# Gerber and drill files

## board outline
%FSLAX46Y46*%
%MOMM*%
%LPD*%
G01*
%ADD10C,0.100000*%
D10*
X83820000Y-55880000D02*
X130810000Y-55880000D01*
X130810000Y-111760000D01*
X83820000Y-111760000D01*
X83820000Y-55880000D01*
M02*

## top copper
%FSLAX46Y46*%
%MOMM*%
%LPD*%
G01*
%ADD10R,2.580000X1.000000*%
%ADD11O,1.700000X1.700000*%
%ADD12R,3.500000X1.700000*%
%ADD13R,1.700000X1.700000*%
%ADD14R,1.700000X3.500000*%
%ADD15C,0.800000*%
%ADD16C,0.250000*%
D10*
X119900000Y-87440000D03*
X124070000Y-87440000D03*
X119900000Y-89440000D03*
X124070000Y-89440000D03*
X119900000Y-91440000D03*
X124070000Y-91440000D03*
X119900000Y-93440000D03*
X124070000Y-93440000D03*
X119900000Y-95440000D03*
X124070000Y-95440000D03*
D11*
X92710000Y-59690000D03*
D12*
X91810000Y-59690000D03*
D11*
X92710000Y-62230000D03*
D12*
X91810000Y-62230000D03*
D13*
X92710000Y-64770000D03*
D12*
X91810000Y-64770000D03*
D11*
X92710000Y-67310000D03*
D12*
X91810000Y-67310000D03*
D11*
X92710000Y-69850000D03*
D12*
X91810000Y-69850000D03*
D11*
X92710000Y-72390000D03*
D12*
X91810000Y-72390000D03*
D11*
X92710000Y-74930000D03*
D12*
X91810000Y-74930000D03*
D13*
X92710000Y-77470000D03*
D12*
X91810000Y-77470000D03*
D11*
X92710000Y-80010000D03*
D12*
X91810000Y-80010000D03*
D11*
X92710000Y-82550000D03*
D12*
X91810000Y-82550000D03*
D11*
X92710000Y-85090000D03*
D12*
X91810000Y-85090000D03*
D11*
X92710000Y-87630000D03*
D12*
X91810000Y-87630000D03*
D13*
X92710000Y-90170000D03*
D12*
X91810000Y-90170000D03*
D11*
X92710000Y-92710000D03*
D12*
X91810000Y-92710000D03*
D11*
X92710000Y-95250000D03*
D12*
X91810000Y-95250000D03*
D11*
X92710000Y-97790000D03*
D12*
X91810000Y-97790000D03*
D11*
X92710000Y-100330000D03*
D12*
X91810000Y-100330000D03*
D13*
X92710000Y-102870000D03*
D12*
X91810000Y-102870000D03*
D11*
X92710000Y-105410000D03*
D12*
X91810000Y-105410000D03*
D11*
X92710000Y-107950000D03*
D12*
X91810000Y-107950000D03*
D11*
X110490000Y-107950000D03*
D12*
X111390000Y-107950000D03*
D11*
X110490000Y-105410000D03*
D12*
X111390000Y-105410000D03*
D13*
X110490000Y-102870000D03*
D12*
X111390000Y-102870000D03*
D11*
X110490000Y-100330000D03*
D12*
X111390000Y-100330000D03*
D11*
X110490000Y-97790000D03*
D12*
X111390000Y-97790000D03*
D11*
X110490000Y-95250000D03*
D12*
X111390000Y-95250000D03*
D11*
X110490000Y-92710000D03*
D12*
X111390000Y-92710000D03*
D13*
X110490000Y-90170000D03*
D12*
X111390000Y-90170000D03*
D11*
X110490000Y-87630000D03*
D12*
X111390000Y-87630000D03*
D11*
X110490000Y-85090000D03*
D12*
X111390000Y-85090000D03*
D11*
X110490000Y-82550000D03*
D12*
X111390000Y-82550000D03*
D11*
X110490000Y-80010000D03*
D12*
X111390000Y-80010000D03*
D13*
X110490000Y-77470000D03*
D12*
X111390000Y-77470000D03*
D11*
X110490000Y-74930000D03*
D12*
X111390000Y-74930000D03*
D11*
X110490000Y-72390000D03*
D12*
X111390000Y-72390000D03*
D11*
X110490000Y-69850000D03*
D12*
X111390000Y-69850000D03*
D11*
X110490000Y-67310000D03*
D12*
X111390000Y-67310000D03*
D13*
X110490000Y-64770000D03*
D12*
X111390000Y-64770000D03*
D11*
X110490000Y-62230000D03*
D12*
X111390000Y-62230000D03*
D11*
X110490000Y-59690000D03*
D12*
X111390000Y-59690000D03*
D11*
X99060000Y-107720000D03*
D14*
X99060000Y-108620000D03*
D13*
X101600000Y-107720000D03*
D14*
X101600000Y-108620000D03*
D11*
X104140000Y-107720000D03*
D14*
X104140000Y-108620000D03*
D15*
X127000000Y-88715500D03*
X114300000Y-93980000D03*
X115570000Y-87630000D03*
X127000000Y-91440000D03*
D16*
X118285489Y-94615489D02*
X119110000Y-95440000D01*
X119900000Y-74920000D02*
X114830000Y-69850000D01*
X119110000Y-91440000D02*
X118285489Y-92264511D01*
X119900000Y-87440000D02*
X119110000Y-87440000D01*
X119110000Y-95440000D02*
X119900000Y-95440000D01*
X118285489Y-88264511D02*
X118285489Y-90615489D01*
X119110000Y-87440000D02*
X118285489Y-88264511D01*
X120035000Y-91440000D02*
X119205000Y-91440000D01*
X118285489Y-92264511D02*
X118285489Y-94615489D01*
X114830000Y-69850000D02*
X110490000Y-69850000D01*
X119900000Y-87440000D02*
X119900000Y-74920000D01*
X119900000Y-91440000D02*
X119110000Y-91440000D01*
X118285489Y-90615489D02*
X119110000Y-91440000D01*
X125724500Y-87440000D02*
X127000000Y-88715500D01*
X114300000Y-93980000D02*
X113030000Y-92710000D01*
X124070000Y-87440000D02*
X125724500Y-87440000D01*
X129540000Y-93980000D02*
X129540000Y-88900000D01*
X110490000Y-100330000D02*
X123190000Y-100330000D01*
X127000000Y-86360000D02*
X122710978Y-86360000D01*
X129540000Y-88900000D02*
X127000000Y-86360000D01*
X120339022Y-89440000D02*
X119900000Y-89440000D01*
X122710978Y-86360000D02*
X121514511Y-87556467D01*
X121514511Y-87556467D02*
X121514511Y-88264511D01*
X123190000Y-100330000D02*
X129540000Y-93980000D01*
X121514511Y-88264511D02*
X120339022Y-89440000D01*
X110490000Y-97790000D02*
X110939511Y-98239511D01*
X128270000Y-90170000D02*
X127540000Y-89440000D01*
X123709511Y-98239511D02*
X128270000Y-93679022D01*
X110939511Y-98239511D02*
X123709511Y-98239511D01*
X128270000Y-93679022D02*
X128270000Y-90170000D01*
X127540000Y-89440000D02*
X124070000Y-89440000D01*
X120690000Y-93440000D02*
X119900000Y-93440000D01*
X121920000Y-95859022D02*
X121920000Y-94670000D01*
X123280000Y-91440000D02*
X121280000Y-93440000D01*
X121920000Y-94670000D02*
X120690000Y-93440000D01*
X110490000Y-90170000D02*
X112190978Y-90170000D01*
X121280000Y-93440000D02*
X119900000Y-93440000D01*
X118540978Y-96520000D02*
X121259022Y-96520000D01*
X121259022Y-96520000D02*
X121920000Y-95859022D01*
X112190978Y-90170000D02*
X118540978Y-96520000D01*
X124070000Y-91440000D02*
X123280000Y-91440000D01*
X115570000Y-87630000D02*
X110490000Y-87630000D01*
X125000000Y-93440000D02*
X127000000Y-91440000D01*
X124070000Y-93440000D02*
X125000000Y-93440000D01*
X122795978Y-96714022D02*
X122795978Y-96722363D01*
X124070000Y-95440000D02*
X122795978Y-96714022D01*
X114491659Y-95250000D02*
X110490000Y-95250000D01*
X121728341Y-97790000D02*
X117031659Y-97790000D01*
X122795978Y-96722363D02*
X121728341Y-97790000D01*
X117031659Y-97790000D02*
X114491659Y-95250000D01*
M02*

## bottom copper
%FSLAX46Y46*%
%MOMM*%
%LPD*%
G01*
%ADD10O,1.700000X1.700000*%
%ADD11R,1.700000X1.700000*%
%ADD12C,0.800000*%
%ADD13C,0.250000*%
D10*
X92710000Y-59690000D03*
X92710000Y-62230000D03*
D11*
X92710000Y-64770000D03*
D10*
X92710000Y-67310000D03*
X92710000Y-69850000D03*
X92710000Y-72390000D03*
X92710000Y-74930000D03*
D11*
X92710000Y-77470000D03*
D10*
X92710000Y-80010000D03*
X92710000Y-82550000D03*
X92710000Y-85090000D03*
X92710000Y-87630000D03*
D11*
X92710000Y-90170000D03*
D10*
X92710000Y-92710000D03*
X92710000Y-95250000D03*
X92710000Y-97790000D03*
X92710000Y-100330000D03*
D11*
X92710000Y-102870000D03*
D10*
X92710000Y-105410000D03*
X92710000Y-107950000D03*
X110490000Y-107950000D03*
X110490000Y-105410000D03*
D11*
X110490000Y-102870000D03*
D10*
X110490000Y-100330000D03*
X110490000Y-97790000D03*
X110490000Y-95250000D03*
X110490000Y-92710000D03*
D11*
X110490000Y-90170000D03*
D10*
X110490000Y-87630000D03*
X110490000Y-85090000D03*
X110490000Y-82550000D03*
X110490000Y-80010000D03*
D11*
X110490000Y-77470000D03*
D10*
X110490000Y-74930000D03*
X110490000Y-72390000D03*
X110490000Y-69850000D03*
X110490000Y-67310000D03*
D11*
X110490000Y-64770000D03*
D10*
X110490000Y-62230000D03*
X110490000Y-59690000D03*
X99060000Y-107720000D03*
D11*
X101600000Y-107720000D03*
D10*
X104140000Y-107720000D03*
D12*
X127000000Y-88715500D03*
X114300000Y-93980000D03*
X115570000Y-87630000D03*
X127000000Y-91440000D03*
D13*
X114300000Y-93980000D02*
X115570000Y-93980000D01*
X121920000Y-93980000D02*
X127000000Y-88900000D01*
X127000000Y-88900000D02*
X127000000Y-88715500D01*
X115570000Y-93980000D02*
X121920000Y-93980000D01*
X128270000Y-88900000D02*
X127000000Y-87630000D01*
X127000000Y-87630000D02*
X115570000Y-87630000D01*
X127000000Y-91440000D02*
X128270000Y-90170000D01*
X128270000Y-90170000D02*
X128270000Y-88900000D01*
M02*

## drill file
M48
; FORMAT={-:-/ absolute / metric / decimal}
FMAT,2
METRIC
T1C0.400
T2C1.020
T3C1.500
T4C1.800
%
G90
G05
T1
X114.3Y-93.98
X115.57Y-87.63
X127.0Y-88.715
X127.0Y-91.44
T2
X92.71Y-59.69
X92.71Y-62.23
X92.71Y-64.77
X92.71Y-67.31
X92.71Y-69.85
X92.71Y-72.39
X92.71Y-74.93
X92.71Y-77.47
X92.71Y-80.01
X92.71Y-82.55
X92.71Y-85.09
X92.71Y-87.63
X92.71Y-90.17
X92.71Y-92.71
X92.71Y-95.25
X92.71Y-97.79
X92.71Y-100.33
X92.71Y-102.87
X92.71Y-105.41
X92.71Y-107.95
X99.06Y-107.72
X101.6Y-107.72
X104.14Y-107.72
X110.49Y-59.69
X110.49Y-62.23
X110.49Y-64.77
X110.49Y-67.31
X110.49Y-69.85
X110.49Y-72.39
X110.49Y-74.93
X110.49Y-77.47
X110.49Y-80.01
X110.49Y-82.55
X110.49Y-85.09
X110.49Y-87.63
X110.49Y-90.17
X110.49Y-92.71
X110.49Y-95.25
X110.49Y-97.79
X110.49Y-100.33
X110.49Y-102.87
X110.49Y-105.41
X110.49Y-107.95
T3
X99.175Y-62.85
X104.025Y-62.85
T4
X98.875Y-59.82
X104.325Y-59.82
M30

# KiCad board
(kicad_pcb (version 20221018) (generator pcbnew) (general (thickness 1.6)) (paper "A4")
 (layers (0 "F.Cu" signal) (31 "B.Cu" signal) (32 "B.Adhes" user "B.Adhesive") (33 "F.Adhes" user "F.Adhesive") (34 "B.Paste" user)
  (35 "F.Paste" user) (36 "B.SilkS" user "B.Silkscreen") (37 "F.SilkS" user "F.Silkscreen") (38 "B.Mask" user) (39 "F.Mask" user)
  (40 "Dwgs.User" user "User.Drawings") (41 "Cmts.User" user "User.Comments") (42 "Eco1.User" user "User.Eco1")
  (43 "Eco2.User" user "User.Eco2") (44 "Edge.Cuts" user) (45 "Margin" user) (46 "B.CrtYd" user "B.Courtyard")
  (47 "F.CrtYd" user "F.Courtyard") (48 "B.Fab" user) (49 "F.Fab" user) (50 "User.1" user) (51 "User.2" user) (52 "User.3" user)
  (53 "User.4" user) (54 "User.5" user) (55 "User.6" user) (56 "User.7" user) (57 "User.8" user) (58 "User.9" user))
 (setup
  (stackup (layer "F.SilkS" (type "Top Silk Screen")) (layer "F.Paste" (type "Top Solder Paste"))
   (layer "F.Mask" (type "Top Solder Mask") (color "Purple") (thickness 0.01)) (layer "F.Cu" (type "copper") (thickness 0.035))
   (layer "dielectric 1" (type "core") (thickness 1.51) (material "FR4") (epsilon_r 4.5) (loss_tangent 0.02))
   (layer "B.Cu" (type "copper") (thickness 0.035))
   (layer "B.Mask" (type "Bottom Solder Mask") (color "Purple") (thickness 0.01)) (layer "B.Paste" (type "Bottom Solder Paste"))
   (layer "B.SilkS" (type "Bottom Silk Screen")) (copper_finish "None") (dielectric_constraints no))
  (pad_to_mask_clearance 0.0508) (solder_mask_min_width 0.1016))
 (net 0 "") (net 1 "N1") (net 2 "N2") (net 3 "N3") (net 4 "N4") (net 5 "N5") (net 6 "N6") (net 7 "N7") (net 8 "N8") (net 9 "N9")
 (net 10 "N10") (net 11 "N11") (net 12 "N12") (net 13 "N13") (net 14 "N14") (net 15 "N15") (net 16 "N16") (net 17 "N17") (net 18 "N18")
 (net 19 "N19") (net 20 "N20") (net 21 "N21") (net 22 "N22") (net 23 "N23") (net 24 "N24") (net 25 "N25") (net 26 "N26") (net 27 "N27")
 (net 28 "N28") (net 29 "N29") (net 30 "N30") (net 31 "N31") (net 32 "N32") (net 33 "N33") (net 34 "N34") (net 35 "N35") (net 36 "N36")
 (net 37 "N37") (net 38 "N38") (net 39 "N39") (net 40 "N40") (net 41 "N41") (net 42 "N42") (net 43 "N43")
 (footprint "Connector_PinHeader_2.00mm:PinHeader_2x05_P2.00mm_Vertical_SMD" (layer "F.Cu") (at 121.985 91.44)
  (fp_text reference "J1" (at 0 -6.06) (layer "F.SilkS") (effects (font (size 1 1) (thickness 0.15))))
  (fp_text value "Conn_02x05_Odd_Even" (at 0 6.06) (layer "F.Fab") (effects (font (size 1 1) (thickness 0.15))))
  (pad "1" smd rect (at -2.085 -4) (size 2.58 1) (layers "F.Cu" "F.Paste" "F.Mask") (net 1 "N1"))
  (pad "2" smd rect (at 2.085 -4) (size 2.58 1) (layers "F.Cu" "F.Paste" "F.Mask") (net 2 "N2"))
  (pad "3" smd rect (at -2.085 -2) (size 2.58 1) (layers "F.Cu" "F.Paste" "F.Mask") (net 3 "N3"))
  (pad "4" smd rect (at 2.085 -2) (size 2.58 1) (layers "F.Cu" "F.Paste" "F.Mask") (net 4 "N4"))
  (pad "5" smd rect (at -2.085 0) (size 2.58 1) (layers "F.Cu" "F.Paste" "F.Mask") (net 1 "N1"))
  (pad "6" smd rect (at 2.085 0) (size 2.58 1) (layers "F.Cu" "F.Paste" "F.Mask") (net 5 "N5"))
  (pad "7" smd rect (at -2.085 2) (size 2.58 1) (layers "F.Cu" "F.Paste" "F.Mask") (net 5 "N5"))
  (pad "8" smd rect (at 2.085 2) (size 2.58 1) (layers "F.Cu" "F.Paste" "F.Mask") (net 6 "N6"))
  (pad "9" smd rect (at -2.085 4) (size 2.58 1) (layers "F.Cu" "F.Paste" "F.Mask") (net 1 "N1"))
  (pad "10" smd rect (at 2.085 4) (size 2.58 1) (layers "F.Cu" "F.Paste" "F.Mask") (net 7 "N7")))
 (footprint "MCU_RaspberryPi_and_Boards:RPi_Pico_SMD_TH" (layer "F.Cu") (at 101.6 83.82)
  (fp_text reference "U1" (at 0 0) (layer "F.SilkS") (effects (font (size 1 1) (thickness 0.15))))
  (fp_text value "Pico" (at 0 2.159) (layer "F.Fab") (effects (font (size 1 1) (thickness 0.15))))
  (pad "" np_thru_hole oval (at -2.725 -24) (size 1.8 1.8) (drill 1.8) (layers "*.Cu" "*.Mask"))
  (pad "" np_thru_hole oval (at -2.425 -20.97) (size 1.5 1.5) (drill 1.5) (layers "*.Cu" "*.Mask"))
  (pad "" np_thru_hole oval (at 2.425 -20.97) (size 1.5 1.5) (drill 1.5) (layers "*.Cu" "*.Mask"))
  (pad "" np_thru_hole oval (at 2.725 -24) (size 1.8 1.8) (drill 1.8) (layers "*.Cu" "*.Mask"))
  (pad "1" thru_hole oval (at -8.89 -24.13) (size 1.7 1.7) (drill 1.02) (layers "*.Cu" "*.Mask") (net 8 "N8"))
  (pad "1" smd rect (at -8.89 -24.13) (size 3.5 1.7) (drill (offset -0.9 0)) (layers "F.Cu" "F.Mask") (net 8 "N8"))
  (pad "2" thru_hole oval (at -8.89 -21.59) (size 1.7 1.7) (drill 1.02) (layers "*.Cu" "*.Mask") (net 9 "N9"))
  (pad "2" smd rect (at -8.89 -21.59) (size 3.5 1.7) (drill (offset -0.9 0)) (layers "F.Cu" "F.Mask") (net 9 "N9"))
  (pad "3" thru_hole rect (at -8.89 -19.05) (size 1.7 1.7) (drill 1.02) (layers "*.Cu" "*.Mask") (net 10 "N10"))
  (pad "3" smd rect (at -8.89 -19.05) (size 3.5 1.7) (drill (offset -0.9 0)) (layers "F.Cu" "F.Mask") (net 10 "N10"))
  (pad "4" thru_hole oval (at -8.89 -16.51) (size 1.7 1.7) (drill 1.02) (layers "*.Cu" "*.Mask") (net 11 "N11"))
  (pad "4" smd rect (at -8.89 -16.51) (size 3.5 1.7) (drill (offset -0.9 0)) (layers "F.Cu" "F.Mask") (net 11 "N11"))
  (pad "5" thru_hole oval (at -8.89 -13.97) (size 1.7 1.7) (drill 1.02) (layers "*.Cu" "*.Mask") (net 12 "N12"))
  (pad "5" smd rect (at -8.89 -13.97) (size 3.5 1.7) (drill (offset -0.9 0)) (layers "F.Cu" "F.Mask") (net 12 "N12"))
  (pad "6" thru_hole oval (at -8.89 -11.43) (size 1.7 1.7) (drill 1.02) (layers "*.Cu" "*.Mask") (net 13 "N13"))
  (pad "6" smd rect (at -8.89 -11.43) (size 3.5 1.7) (drill (offset -0.9 0)) (layers "F.Cu" "F.Mask") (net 13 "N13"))
  (pad "7" thru_hole oval (at -8.89 -8.89) (size 1.7 1.7) (drill 1.02) (layers "*.Cu" "*.Mask") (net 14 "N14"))
  (pad "7" smd rect (at -8.89 -8.89) (size 3.5 1.7) (drill (offset -0.9 0)) (layers "F.Cu" "F.Mask") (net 14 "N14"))
  (pad "8" thru_hole rect (at -8.89 -6.35) (size 1.7 1.7) (drill 1.02) (layers "*.Cu" "*.Mask") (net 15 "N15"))
  (pad "8" smd rect (at -8.89 -6.35) (size 3.5 1.7) (drill (offset -0.9 0)) (layers "F.Cu" "F.Mask") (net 15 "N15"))
  (pad "9" thru_hole oval (at -8.89 -3.81) (size 1.7 1.7) (drill 1.02) (layers "*.Cu" "*.Mask") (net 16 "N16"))
  (pad "9" smd rect (at -8.89 -3.81) (size 3.5 1.7) (drill (offset -0.9 0)) (layers "F.Cu" "F.Mask") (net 16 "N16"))
  (pad "10" thru_hole oval (at -8.89 -1.27) (size 1.7 1.7) (drill 1.02) (layers "*.Cu" "*.Mask") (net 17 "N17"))
  (pad "10" smd rect (at -8.89 -1.27) (size 3.5 1.7) (drill (offset -0.9 0)) (layers "F.Cu" "F.Mask") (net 17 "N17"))
  (pad "11" thru_hole oval (at -8.89 1.27) (size 1.7 1.7) (drill 1.02) (layers "*.Cu" "*.Mask") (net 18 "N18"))
  (pad "11" smd rect (at -8.89 1.27) (size 3.5 1.7) (drill (offset -0.9 0)) (layers "F.Cu" "F.Mask") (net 18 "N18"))
  (pad "12" thru_hole oval (at -8.89 3.81) (size 1.7 1.7) (drill 1.02) (layers "*.Cu" "*.Mask") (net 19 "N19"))
  (pad "12" smd rect (at -8.89 3.81) (size 3.5 1.7) (drill (offset -0.9 0)) (layers "F.Cu" "F.Mask") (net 19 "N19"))
  (pad "13" thru_hole rect (at -8.89 6.35) (size 1.7 1.7) (drill 1.02) (layers "*.Cu" "*.Mask") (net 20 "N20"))
  (pad "13" smd rect (at -8.89 6.35) (size 3.5 1.7) (drill (offset -0.9 0)) (layers "F.Cu" "F.Mask") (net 20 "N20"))
  (pad "14" thru_hole oval (at -8.89 8.89) (size 1.7 1.7) (drill 1.02) (layers "*.Cu" "*.Mask") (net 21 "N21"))
  (pad "14" smd rect (at -8.89 8.89) (size 3.5 1.7) (drill (offset -0.9 0)) (layers "F.Cu" "F.Mask") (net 21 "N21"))
  (pad "15" thru_hole oval (at -8.89 11.43) (size 1.7 1.7) (drill 1.02) (layers "*.Cu" "*.Mask") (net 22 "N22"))
  (pad "15" smd rect (at -8.89 11.43) (size 3.5 1.7) (drill (offset -0.9 0)) (layers "F.Cu" "F.Mask") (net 22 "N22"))
  (pad "16" thru_hole oval (at -8.89 13.97) (size 1.7 1.7) (drill 1.02) (layers "*.Cu" "*.Mask") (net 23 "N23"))
  (pad "16" smd rect (at -8.89 13.97) (size 3.5 1.7) (drill (offset -0.9 0)) (layers "F.Cu" "F.Mask") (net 23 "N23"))
  (pad "17" thru_hole oval (at -8.89 16.51) (size 1.7 1.7) (drill 1.02) (layers "*.Cu" "*.Mask") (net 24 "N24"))
  (pad "17" smd rect (at -8.89 16.51) (size 3.5 1.7) (drill (offset -0.9 0)) (layers "F.Cu" "F.Mask") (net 24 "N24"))
  (pad "18" thru_hole rect (at -8.89 19.05) (size 1.7 1.7) (drill 1.02) (layers "*.Cu" "*.Mask") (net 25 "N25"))
  (pad "18" smd rect (at -8.89 19.05) (size 3.5 1.7) (drill (offset -0.9 0)) (layers "F.Cu" "F.Mask") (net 25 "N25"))
  (pad "19" thru_hole oval (at -8.89 21.59) (size 1.7 1.7) (drill 1.02) (layers "*.Cu" "*.Mask") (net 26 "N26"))
  (pad "19" smd rect (at -8.89 21.59) (size 3.5 1.7) (drill (offset -0.9 0)) (layers "F.Cu" "F.Mask") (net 26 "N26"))
  (pad "20" thru_hole oval (at -8.89 24.13) (size 1.7 1.7) (drill 1.02) (layers "*.Cu" "*.Mask") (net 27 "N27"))
  (pad "20" smd rect (at -8.89 24.13) (size 3.5 1.7) (drill (offset -0.9 0)) (layers "F.Cu" "F.Mask") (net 27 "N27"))
  (pad "21" thru_hole oval (at 8.89 24.13) (size 1.7 1.7) (drill 1.02) (layers "*.Cu" "*.Mask") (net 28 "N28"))
  (pad "21" smd rect (at 8.89 24.13) (size 3.5 1.7) (drill (offset 0.9 0)) (layers "F.Cu" "F.Mask") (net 28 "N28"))
  (pad "22" thru_hole oval (at 8.89 21.59) (size 1.7 1.7) (drill 1.02) (layers "*.Cu" "*.Mask") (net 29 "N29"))
  (pad "22" smd rect (at 8.89 21.59) (size 3.5 1.7) (drill (offset 0.9 0)) (layers "F.Cu" "F.Mask") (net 29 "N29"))
  (pad "23" thru_hole rect (at 8.89 19.05) (size 1.7 1.7) (drill 1.02) (layers "*.Cu" "*.Mask") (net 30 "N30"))
  (pad "23" smd rect (at 8.89 19.05) (size 3.5 1.7) (drill (offset 0.9 0)) (layers "F.Cu" "F.Mask") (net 30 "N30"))
  (pad "24" thru_hole oval (at 8.89 16.51) (size 1.7 1.7) (drill 1.02) (layers "*.Cu" "*.Mask") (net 3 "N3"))
  (pad "24" smd rect (at 8.89 16.51) (size 3.5 1.7) (drill (offset 0.9 0)) (layers "F.Cu" "F.Mask") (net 3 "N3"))
  (pad "25" thru_hole oval (at 8.89 13.97) (size 1.7 1.7) (drill 1.02) (layers "*.Cu" "*.Mask") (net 4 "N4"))
  (pad "25" smd rect (at 8.89 13.97) (size 3.5 1.7) (drill (offset 0.9 0)) (layers "F.Cu" "F.Mask") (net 4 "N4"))
  (pad "26" thru_hole oval (at 8.89 11.43) (size 1.7 1.7) (drill 1.02) (layers "*.Cu" "*.Mask") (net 7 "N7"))
  (pad "26" smd rect (at 8.89 11.43) (size 3.5 1.7) (drill (offset 0.9 0)) (layers "F.Cu" "F.Mask") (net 7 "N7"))
  (pad "27" thru_hole oval (at 8.89 8.89) (size 1.7 1.7) (drill 1.02) (layers "*.Cu" "*.Mask") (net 2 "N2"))
  (pad "27" smd rect (at 8.89 8.89) (size 3.5 1.7) (drill (offset 0.9 0)) (layers "F.Cu" "F.Mask") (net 2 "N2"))
  (pad "28" thru_hole rect (at 8.89 6.35) (size 1.7 1.7) (drill 1.02) (layers "*.Cu" "*.Mask") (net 5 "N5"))
  (pad "28" smd rect (at 8.89 6.35) (size 3.5 1.7) (drill (offset 0.9 0)) (layers "F.Cu" "F.Mask") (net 5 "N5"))
  (pad "29" thru_hole oval (at 8.89 3.81) (size 1.7 1.7) (drill 1.02) (layers "*.Cu" "*.Mask") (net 6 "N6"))
  (pad "29" smd rect (at 8.89 3.81) (size 3.5 1.7) (drill (offset 0.9 0)) (layers "F.Cu" "F.Mask") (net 6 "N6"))
  (pad "30" thru_hole oval (at 8.89 1.27) (size 1.7 1.7) (drill 1.02) (layers "*.Cu" "*.Mask") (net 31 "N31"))
  (pad "30" smd rect (at 8.89 1.27) (size 3.5 1.7) (drill (offset 0.9 0)) (layers "F.Cu" "F.Mask") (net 31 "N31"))
  (pad "31" thru_hole oval (at 8.89 -1.27) (size 1.7 1.7) (drill 1.02) (layers "*.Cu" "*.Mask") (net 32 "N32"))
  (pad "31" smd rect (at 8.89 -1.27) (size 3.5 1.7) (drill (offset 0.9 0)) (layers "F.Cu" "F.Mask") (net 32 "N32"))
  (pad "32" thru_hole oval (at 8.89 -3.81) (size 1.7 1.7) (drill 1.02) (layers "*.Cu" "*.Mask") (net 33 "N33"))
  (pad "32" smd rect (at 8.89 -3.81) (size 3.5 1.7) (drill (offset 0.9 0)) (layers "F.Cu" "F.Mask") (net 33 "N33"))
  (pad "33" thru_hole rect (at 8.89 -6.35) (size 1.7 1.7) (drill 1.02) (layers "*.Cu" "*.Mask") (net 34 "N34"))
  (pad "33" smd rect (at 8.89 -6.35) (size 3.5 1.7) (drill (offset 0.9 0)) (layers "F.Cu" "F.Mask") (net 34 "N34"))
  (pad "34" thru_hole oval (at 8.89 -8.89) (size 1.7 1.7) (drill 1.02) (layers "*.Cu" "*.Mask") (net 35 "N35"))
  (pad "34" smd rect (at 8.89 -8.89) (size 3.5 1.7) (drill (offset 0.9 0)) (layers "F.Cu" "F.Mask") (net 35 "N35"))
  (pad "35" thru_hole oval (at 8.89 -11.43) (size 1.7 1.7) (drill 1.02) (layers "*.Cu" "*.Mask") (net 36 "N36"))
  (pad "35" smd rect (at 8.89 -11.43) (size 3.5 1.7) (drill (offset 0.9 0)) (layers "F.Cu" "F.Mask") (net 36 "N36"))
  (pad "36" thru_hole oval (at 8.89 -13.97) (size 1.7 1.7) (drill 1.02) (layers "*.Cu" "*.Mask") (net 1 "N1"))
  (pad "36" smd rect (at 8.89 -13.97) (size 3.5 1.7) (drill (offset 0.9 0)) (layers "F.Cu" "F.Mask") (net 1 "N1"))
  (pad "37" thru_hole oval (at 8.89 -16.51) (size 1.7 1.7) (drill 1.02) (layers "*.Cu" "*.Mask") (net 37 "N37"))
  (pad "37" smd rect (at 8.89 -16.51) (size 3.5 1.7) (drill (offset 0.9 0)) (layers "F.Cu" "F.Mask") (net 37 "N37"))
  (pad "38" thru_hole rect (at 8.89 -19.05) (size 1.7 1.7) (drill 1.02) (layers "*.Cu" "*.Mask") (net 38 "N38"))
  (pad "38" smd rect (at 8.89 -19.05) (size 3.5 1.7) (drill (offset 0.9 0)) (layers "F.Cu" "F.Mask") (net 38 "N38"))
  (pad "39" thru_hole oval (at 8.89 -21.59) (size 1.7 1.7) (drill 1.02) (layers "*.Cu" "*.Mask") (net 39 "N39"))
  (pad "39" smd rect (at 8.89 -21.59) (size 3.5 1.7) (drill (offset 0.9 0)) (layers "F.Cu" "F.Mask") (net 39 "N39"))
  (pad "40" thru_hole oval (at 8.89 -24.13) (size 1.7 1.7) (drill 1.02) (layers "*.Cu" "*.Mask") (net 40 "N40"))
  (pad "40" smd rect (at 8.89 -24.13) (size 3.5 1.7) (drill (offset 0.9 0)) (layers "F.Cu" "F.Mask") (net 40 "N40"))
  (pad "41" thru_hole oval (at -2.54 23.9) (size 1.7 1.7) (drill 1.02) (layers "*.Cu" "*.Mask") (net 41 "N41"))
  (pad "41" smd rect (at -2.54 23.9 90) (size 3.5 1.7) (drill (offset -0.9 0)) (layers "F.Cu" "F.Mask") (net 41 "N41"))
  (pad "42" thru_hole rect (at 0 23.9) (size 1.7 1.7) (drill 1.02) (layers "*.Cu" "*.Mask") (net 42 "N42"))
  (pad "42" smd rect (at 0 23.9 90) (size 3.5 1.7) (drill (offset -0.9 0)) (layers "F.Cu" "F.Mask") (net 42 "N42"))
  (pad "43" thru_hole oval (at 2.54 23.9) (size 1.7 1.7) (drill 1.02) (layers "*.Cu" "*.Mask") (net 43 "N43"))
  (pad "43" smd rect (at 2.54 23.9 90) (size 3.5 1.7) (drill (offset -0.9 0)) (layers "F.Cu" "F.Mask") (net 43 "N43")))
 (gr_rect (start 83.82 55.88) (end 130.81 111.76) (stroke (width 0.1) (type solid)) (fill none) (layer "Edge.Cuts"))
 (segment (start 118.285489 94.615489) (end 119.11 95.44) (width 0.25) (layer "F.Cu") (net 1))
 (segment (start 119.9 74.92) (end 114.83 69.85) (width 0.25) (layer "F.Cu") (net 1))
 (segment (start 119.11 91.44) (end 118.285489 92.264511) (width 0.25) (layer "F.Cu") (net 1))
 (segment (start 119.9 87.44) (end 119.11 87.44) (width 0.25) (layer "F.Cu") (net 1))
 (segment (start 119.11 95.44) (end 119.9 95.44) (width 0.25) (layer "F.Cu") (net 1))
 (segment (start 118.285489 88.264511) (end 118.285489 90.615489) (width 0.25) (layer "F.Cu") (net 1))
 (segment (start 119.11 87.44) (end 118.285489 88.264511) (width 0.25) (layer "F.Cu") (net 1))
 (segment (start 120.035 91.44) (end 119.205 91.44) (width 0.25) (layer "F.Cu") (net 1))
 (segment (start 118.285489 92.264511) (end 118.285489 94.615489) (width 0.25) (layer "F.Cu") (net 1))
 (segment (start 114.83 69.85) (end 110.49 69.85) (width 0.25) (layer "F.Cu") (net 1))
 (segment (start 119.9 87.44) (end 119.9 74.92) (width 0.25) (layer "F.Cu") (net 1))
 (segment (start 119.9 91.44) (end 119.11 91.44) (width 0.25) (layer "F.Cu") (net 1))
 (segment (start 118.285489 90.615489) (end 119.11 91.44) (width 0.25) (layer "F.Cu") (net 1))
 (segment (start 125.7245 87.44) (end 127 88.7155) (width 0.25) (layer "F.Cu") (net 2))
 (segment (start 114.3 93.98) (end 113.03 92.71) (width 0.25) (layer "F.Cu") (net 2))
 (segment (start 124.07 87.44) (end 125.7245 87.44) (width 0.25) (layer "F.Cu") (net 2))
 (via (at 127 88.7155) (size 0.8) (drill 0.4) (layers "F.Cu" "B.Cu") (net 2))
 (via (at 114.3 93.98) (size 0.8) (drill 0.4) (layers "F.Cu" "B.Cu") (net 2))
 (segment (start 114.3 93.98) (end 115.57 93.98) (width 0.25) (layer "B.Cu") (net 2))
 (segment (start 121.92 93.98) (end 127 88.9) (width 0.25) (layer "B.Cu") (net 2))
 (segment (start 127 88.9) (end 127 88.7155) (width 0.25) (layer "B.Cu") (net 2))
 (segment (start 115.57 93.98) (end 121.92 93.98) (width 0.25) (layer "B.Cu") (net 2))
 (segment (start 129.54 93.98) (end 129.54 88.9) (width 0.25) (layer "F.Cu") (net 3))
 (segment (start 110.49 100.33) (end 123.19 100.33) (width 0.25) (layer "F.Cu") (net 3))
 (segment (start 127 86.36) (end 122.710978 86.36) (width 0.25) (layer "F.Cu") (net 3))
 (segment (start 129.54 88.9) (end 127 86.36) (width 0.25) (layer "F.Cu") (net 3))
 (segment (start 120.339022 89.44) (end 119.9 89.44) (width 0.25) (layer "F.Cu") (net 3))
 (segment (start 122.710978 86.36) (end 121.514511 87.556467) (width 0.25) (layer "F.Cu") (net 3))
 (segment (start 121.514511 87.556467) (end 121.514511 88.264511) (width 0.25) (layer "F.Cu") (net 3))
 (segment (start 123.19 100.33) (end 129.54 93.98) (width 0.25) (layer "F.Cu") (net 3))
 (segment (start 121.514511 88.264511) (end 120.339022 89.44) (width 0.25) (layer "F.Cu") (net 3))
 (segment (start 110.49 97.79) (end 110.939511 98.239511) (width 0.25) (layer "F.Cu") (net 4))
 (segment (start 128.27 90.17) (end 127.54 89.44) (width 0.25) (layer "F.Cu") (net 4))
 (segment (start 123.709511 98.239511) (end 128.27 93.679022) (width 0.25) (layer "F.Cu") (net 4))
 (segment (start 110.939511 98.239511) (end 123.709511 98.239511) (width 0.25) (layer "F.Cu") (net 4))
 (segment (start 128.27 93.679022) (end 128.27 90.17) (width 0.25) (layer "F.Cu") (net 4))
 (segment (start 127.54 89.44) (end 124.07 89.44) (width 0.25) (layer "F.Cu") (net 4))
 (segment (start 120.69 93.44) (end 119.9 93.44) (width 0.25) (layer "F.Cu") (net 5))
 (segment (start 121.92 95.859022) (end 121.92 94.67) (width 0.25) (layer "F.Cu") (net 5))
 (segment (start 123.28 91.44) (end 121.28 93.44) (width 0.25) (layer "F.Cu") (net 5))
 (segment (start 121.92 94.67) (end 120.69 93.44) (width 0.25) (layer "F.Cu") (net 5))
 (segment (start 110.49 90.17) (end 112.190978 90.17) (width 0.25) (layer "F.Cu") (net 5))
 (segment (start 121.28 93.44) (end 119.9 93.44) (width 0.25) (layer "F.Cu") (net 5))
 (segment (start 118.540978 96.52) (end 121.259022 96.52) (width 0.25) (layer "F.Cu") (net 5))
 (segment (start 121.259022 96.52) (end 121.92 95.859022) (width 0.25) (layer "F.Cu") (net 5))
 (segment (start 112.190978 90.17) (end 118.540978 96.52) (width 0.25) (layer "F.Cu") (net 5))
 (segment (start 124.07 91.44) (end 123.28 91.44) (width 0.25) (layer "F.Cu") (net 5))
 (segment (start 115.57 87.63) (end 110.49 87.63) (width 0.25) (layer "F.Cu") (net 6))
 (segment (start 125 93.44) (end 127 91.44) (width 0.25) (layer "F.Cu") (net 6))
 (segment (start 124.07 93.44) (end 125 93.44) (width 0.25) (layer "F.Cu") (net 6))
 (via (at 115.57 87.63) (size 0.8) (drill 0.4) (layers "F.Cu" "B.Cu") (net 6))
 (via (at 127 91.44) (size 0.8) (drill 0.4) (layers "F.Cu" "B.Cu") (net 6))
 (segment (start 128.27 88.9) (end 127 87.63) (width 0.25) (layer "B.Cu") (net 6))
 (segment (start 127 87.63) (end 115.57 87.63) (width 0.25) (layer "B.Cu") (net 6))
 (segment (start 127 91.44) (end 128.27 90.17) (width 0.25) (layer "B.Cu") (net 6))
 (segment (start 128.27 90.17) (end 128.27 88.9) (width 0.25) (layer "B.Cu") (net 6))
 (segment (start 122.795978 96.714022) (end 122.795978 96.722363) (width 0.25) (layer "F.Cu") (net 7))
 (segment (start 124.07 95.44) (end 122.795978 96.714022) (width 0.25) (layer "F.Cu") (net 7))
 (segment (start 114.491659 95.25) (end 110.49 95.25) (width 0.25) (layer "F.Cu") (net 7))
 (segment (start 121.728341 97.79) (end 117.031659 97.79) (width 0.25) (layer "F.Cu") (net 7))
 (segment (start 122.795978 96.722363) (end 121.728341 97.79) (width 0.25) (layer "F.Cu") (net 7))
 (segment (start 117.031659 97.79) (end 114.491659 95.25) (width 0.25) (layer "F.Cu") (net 7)))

